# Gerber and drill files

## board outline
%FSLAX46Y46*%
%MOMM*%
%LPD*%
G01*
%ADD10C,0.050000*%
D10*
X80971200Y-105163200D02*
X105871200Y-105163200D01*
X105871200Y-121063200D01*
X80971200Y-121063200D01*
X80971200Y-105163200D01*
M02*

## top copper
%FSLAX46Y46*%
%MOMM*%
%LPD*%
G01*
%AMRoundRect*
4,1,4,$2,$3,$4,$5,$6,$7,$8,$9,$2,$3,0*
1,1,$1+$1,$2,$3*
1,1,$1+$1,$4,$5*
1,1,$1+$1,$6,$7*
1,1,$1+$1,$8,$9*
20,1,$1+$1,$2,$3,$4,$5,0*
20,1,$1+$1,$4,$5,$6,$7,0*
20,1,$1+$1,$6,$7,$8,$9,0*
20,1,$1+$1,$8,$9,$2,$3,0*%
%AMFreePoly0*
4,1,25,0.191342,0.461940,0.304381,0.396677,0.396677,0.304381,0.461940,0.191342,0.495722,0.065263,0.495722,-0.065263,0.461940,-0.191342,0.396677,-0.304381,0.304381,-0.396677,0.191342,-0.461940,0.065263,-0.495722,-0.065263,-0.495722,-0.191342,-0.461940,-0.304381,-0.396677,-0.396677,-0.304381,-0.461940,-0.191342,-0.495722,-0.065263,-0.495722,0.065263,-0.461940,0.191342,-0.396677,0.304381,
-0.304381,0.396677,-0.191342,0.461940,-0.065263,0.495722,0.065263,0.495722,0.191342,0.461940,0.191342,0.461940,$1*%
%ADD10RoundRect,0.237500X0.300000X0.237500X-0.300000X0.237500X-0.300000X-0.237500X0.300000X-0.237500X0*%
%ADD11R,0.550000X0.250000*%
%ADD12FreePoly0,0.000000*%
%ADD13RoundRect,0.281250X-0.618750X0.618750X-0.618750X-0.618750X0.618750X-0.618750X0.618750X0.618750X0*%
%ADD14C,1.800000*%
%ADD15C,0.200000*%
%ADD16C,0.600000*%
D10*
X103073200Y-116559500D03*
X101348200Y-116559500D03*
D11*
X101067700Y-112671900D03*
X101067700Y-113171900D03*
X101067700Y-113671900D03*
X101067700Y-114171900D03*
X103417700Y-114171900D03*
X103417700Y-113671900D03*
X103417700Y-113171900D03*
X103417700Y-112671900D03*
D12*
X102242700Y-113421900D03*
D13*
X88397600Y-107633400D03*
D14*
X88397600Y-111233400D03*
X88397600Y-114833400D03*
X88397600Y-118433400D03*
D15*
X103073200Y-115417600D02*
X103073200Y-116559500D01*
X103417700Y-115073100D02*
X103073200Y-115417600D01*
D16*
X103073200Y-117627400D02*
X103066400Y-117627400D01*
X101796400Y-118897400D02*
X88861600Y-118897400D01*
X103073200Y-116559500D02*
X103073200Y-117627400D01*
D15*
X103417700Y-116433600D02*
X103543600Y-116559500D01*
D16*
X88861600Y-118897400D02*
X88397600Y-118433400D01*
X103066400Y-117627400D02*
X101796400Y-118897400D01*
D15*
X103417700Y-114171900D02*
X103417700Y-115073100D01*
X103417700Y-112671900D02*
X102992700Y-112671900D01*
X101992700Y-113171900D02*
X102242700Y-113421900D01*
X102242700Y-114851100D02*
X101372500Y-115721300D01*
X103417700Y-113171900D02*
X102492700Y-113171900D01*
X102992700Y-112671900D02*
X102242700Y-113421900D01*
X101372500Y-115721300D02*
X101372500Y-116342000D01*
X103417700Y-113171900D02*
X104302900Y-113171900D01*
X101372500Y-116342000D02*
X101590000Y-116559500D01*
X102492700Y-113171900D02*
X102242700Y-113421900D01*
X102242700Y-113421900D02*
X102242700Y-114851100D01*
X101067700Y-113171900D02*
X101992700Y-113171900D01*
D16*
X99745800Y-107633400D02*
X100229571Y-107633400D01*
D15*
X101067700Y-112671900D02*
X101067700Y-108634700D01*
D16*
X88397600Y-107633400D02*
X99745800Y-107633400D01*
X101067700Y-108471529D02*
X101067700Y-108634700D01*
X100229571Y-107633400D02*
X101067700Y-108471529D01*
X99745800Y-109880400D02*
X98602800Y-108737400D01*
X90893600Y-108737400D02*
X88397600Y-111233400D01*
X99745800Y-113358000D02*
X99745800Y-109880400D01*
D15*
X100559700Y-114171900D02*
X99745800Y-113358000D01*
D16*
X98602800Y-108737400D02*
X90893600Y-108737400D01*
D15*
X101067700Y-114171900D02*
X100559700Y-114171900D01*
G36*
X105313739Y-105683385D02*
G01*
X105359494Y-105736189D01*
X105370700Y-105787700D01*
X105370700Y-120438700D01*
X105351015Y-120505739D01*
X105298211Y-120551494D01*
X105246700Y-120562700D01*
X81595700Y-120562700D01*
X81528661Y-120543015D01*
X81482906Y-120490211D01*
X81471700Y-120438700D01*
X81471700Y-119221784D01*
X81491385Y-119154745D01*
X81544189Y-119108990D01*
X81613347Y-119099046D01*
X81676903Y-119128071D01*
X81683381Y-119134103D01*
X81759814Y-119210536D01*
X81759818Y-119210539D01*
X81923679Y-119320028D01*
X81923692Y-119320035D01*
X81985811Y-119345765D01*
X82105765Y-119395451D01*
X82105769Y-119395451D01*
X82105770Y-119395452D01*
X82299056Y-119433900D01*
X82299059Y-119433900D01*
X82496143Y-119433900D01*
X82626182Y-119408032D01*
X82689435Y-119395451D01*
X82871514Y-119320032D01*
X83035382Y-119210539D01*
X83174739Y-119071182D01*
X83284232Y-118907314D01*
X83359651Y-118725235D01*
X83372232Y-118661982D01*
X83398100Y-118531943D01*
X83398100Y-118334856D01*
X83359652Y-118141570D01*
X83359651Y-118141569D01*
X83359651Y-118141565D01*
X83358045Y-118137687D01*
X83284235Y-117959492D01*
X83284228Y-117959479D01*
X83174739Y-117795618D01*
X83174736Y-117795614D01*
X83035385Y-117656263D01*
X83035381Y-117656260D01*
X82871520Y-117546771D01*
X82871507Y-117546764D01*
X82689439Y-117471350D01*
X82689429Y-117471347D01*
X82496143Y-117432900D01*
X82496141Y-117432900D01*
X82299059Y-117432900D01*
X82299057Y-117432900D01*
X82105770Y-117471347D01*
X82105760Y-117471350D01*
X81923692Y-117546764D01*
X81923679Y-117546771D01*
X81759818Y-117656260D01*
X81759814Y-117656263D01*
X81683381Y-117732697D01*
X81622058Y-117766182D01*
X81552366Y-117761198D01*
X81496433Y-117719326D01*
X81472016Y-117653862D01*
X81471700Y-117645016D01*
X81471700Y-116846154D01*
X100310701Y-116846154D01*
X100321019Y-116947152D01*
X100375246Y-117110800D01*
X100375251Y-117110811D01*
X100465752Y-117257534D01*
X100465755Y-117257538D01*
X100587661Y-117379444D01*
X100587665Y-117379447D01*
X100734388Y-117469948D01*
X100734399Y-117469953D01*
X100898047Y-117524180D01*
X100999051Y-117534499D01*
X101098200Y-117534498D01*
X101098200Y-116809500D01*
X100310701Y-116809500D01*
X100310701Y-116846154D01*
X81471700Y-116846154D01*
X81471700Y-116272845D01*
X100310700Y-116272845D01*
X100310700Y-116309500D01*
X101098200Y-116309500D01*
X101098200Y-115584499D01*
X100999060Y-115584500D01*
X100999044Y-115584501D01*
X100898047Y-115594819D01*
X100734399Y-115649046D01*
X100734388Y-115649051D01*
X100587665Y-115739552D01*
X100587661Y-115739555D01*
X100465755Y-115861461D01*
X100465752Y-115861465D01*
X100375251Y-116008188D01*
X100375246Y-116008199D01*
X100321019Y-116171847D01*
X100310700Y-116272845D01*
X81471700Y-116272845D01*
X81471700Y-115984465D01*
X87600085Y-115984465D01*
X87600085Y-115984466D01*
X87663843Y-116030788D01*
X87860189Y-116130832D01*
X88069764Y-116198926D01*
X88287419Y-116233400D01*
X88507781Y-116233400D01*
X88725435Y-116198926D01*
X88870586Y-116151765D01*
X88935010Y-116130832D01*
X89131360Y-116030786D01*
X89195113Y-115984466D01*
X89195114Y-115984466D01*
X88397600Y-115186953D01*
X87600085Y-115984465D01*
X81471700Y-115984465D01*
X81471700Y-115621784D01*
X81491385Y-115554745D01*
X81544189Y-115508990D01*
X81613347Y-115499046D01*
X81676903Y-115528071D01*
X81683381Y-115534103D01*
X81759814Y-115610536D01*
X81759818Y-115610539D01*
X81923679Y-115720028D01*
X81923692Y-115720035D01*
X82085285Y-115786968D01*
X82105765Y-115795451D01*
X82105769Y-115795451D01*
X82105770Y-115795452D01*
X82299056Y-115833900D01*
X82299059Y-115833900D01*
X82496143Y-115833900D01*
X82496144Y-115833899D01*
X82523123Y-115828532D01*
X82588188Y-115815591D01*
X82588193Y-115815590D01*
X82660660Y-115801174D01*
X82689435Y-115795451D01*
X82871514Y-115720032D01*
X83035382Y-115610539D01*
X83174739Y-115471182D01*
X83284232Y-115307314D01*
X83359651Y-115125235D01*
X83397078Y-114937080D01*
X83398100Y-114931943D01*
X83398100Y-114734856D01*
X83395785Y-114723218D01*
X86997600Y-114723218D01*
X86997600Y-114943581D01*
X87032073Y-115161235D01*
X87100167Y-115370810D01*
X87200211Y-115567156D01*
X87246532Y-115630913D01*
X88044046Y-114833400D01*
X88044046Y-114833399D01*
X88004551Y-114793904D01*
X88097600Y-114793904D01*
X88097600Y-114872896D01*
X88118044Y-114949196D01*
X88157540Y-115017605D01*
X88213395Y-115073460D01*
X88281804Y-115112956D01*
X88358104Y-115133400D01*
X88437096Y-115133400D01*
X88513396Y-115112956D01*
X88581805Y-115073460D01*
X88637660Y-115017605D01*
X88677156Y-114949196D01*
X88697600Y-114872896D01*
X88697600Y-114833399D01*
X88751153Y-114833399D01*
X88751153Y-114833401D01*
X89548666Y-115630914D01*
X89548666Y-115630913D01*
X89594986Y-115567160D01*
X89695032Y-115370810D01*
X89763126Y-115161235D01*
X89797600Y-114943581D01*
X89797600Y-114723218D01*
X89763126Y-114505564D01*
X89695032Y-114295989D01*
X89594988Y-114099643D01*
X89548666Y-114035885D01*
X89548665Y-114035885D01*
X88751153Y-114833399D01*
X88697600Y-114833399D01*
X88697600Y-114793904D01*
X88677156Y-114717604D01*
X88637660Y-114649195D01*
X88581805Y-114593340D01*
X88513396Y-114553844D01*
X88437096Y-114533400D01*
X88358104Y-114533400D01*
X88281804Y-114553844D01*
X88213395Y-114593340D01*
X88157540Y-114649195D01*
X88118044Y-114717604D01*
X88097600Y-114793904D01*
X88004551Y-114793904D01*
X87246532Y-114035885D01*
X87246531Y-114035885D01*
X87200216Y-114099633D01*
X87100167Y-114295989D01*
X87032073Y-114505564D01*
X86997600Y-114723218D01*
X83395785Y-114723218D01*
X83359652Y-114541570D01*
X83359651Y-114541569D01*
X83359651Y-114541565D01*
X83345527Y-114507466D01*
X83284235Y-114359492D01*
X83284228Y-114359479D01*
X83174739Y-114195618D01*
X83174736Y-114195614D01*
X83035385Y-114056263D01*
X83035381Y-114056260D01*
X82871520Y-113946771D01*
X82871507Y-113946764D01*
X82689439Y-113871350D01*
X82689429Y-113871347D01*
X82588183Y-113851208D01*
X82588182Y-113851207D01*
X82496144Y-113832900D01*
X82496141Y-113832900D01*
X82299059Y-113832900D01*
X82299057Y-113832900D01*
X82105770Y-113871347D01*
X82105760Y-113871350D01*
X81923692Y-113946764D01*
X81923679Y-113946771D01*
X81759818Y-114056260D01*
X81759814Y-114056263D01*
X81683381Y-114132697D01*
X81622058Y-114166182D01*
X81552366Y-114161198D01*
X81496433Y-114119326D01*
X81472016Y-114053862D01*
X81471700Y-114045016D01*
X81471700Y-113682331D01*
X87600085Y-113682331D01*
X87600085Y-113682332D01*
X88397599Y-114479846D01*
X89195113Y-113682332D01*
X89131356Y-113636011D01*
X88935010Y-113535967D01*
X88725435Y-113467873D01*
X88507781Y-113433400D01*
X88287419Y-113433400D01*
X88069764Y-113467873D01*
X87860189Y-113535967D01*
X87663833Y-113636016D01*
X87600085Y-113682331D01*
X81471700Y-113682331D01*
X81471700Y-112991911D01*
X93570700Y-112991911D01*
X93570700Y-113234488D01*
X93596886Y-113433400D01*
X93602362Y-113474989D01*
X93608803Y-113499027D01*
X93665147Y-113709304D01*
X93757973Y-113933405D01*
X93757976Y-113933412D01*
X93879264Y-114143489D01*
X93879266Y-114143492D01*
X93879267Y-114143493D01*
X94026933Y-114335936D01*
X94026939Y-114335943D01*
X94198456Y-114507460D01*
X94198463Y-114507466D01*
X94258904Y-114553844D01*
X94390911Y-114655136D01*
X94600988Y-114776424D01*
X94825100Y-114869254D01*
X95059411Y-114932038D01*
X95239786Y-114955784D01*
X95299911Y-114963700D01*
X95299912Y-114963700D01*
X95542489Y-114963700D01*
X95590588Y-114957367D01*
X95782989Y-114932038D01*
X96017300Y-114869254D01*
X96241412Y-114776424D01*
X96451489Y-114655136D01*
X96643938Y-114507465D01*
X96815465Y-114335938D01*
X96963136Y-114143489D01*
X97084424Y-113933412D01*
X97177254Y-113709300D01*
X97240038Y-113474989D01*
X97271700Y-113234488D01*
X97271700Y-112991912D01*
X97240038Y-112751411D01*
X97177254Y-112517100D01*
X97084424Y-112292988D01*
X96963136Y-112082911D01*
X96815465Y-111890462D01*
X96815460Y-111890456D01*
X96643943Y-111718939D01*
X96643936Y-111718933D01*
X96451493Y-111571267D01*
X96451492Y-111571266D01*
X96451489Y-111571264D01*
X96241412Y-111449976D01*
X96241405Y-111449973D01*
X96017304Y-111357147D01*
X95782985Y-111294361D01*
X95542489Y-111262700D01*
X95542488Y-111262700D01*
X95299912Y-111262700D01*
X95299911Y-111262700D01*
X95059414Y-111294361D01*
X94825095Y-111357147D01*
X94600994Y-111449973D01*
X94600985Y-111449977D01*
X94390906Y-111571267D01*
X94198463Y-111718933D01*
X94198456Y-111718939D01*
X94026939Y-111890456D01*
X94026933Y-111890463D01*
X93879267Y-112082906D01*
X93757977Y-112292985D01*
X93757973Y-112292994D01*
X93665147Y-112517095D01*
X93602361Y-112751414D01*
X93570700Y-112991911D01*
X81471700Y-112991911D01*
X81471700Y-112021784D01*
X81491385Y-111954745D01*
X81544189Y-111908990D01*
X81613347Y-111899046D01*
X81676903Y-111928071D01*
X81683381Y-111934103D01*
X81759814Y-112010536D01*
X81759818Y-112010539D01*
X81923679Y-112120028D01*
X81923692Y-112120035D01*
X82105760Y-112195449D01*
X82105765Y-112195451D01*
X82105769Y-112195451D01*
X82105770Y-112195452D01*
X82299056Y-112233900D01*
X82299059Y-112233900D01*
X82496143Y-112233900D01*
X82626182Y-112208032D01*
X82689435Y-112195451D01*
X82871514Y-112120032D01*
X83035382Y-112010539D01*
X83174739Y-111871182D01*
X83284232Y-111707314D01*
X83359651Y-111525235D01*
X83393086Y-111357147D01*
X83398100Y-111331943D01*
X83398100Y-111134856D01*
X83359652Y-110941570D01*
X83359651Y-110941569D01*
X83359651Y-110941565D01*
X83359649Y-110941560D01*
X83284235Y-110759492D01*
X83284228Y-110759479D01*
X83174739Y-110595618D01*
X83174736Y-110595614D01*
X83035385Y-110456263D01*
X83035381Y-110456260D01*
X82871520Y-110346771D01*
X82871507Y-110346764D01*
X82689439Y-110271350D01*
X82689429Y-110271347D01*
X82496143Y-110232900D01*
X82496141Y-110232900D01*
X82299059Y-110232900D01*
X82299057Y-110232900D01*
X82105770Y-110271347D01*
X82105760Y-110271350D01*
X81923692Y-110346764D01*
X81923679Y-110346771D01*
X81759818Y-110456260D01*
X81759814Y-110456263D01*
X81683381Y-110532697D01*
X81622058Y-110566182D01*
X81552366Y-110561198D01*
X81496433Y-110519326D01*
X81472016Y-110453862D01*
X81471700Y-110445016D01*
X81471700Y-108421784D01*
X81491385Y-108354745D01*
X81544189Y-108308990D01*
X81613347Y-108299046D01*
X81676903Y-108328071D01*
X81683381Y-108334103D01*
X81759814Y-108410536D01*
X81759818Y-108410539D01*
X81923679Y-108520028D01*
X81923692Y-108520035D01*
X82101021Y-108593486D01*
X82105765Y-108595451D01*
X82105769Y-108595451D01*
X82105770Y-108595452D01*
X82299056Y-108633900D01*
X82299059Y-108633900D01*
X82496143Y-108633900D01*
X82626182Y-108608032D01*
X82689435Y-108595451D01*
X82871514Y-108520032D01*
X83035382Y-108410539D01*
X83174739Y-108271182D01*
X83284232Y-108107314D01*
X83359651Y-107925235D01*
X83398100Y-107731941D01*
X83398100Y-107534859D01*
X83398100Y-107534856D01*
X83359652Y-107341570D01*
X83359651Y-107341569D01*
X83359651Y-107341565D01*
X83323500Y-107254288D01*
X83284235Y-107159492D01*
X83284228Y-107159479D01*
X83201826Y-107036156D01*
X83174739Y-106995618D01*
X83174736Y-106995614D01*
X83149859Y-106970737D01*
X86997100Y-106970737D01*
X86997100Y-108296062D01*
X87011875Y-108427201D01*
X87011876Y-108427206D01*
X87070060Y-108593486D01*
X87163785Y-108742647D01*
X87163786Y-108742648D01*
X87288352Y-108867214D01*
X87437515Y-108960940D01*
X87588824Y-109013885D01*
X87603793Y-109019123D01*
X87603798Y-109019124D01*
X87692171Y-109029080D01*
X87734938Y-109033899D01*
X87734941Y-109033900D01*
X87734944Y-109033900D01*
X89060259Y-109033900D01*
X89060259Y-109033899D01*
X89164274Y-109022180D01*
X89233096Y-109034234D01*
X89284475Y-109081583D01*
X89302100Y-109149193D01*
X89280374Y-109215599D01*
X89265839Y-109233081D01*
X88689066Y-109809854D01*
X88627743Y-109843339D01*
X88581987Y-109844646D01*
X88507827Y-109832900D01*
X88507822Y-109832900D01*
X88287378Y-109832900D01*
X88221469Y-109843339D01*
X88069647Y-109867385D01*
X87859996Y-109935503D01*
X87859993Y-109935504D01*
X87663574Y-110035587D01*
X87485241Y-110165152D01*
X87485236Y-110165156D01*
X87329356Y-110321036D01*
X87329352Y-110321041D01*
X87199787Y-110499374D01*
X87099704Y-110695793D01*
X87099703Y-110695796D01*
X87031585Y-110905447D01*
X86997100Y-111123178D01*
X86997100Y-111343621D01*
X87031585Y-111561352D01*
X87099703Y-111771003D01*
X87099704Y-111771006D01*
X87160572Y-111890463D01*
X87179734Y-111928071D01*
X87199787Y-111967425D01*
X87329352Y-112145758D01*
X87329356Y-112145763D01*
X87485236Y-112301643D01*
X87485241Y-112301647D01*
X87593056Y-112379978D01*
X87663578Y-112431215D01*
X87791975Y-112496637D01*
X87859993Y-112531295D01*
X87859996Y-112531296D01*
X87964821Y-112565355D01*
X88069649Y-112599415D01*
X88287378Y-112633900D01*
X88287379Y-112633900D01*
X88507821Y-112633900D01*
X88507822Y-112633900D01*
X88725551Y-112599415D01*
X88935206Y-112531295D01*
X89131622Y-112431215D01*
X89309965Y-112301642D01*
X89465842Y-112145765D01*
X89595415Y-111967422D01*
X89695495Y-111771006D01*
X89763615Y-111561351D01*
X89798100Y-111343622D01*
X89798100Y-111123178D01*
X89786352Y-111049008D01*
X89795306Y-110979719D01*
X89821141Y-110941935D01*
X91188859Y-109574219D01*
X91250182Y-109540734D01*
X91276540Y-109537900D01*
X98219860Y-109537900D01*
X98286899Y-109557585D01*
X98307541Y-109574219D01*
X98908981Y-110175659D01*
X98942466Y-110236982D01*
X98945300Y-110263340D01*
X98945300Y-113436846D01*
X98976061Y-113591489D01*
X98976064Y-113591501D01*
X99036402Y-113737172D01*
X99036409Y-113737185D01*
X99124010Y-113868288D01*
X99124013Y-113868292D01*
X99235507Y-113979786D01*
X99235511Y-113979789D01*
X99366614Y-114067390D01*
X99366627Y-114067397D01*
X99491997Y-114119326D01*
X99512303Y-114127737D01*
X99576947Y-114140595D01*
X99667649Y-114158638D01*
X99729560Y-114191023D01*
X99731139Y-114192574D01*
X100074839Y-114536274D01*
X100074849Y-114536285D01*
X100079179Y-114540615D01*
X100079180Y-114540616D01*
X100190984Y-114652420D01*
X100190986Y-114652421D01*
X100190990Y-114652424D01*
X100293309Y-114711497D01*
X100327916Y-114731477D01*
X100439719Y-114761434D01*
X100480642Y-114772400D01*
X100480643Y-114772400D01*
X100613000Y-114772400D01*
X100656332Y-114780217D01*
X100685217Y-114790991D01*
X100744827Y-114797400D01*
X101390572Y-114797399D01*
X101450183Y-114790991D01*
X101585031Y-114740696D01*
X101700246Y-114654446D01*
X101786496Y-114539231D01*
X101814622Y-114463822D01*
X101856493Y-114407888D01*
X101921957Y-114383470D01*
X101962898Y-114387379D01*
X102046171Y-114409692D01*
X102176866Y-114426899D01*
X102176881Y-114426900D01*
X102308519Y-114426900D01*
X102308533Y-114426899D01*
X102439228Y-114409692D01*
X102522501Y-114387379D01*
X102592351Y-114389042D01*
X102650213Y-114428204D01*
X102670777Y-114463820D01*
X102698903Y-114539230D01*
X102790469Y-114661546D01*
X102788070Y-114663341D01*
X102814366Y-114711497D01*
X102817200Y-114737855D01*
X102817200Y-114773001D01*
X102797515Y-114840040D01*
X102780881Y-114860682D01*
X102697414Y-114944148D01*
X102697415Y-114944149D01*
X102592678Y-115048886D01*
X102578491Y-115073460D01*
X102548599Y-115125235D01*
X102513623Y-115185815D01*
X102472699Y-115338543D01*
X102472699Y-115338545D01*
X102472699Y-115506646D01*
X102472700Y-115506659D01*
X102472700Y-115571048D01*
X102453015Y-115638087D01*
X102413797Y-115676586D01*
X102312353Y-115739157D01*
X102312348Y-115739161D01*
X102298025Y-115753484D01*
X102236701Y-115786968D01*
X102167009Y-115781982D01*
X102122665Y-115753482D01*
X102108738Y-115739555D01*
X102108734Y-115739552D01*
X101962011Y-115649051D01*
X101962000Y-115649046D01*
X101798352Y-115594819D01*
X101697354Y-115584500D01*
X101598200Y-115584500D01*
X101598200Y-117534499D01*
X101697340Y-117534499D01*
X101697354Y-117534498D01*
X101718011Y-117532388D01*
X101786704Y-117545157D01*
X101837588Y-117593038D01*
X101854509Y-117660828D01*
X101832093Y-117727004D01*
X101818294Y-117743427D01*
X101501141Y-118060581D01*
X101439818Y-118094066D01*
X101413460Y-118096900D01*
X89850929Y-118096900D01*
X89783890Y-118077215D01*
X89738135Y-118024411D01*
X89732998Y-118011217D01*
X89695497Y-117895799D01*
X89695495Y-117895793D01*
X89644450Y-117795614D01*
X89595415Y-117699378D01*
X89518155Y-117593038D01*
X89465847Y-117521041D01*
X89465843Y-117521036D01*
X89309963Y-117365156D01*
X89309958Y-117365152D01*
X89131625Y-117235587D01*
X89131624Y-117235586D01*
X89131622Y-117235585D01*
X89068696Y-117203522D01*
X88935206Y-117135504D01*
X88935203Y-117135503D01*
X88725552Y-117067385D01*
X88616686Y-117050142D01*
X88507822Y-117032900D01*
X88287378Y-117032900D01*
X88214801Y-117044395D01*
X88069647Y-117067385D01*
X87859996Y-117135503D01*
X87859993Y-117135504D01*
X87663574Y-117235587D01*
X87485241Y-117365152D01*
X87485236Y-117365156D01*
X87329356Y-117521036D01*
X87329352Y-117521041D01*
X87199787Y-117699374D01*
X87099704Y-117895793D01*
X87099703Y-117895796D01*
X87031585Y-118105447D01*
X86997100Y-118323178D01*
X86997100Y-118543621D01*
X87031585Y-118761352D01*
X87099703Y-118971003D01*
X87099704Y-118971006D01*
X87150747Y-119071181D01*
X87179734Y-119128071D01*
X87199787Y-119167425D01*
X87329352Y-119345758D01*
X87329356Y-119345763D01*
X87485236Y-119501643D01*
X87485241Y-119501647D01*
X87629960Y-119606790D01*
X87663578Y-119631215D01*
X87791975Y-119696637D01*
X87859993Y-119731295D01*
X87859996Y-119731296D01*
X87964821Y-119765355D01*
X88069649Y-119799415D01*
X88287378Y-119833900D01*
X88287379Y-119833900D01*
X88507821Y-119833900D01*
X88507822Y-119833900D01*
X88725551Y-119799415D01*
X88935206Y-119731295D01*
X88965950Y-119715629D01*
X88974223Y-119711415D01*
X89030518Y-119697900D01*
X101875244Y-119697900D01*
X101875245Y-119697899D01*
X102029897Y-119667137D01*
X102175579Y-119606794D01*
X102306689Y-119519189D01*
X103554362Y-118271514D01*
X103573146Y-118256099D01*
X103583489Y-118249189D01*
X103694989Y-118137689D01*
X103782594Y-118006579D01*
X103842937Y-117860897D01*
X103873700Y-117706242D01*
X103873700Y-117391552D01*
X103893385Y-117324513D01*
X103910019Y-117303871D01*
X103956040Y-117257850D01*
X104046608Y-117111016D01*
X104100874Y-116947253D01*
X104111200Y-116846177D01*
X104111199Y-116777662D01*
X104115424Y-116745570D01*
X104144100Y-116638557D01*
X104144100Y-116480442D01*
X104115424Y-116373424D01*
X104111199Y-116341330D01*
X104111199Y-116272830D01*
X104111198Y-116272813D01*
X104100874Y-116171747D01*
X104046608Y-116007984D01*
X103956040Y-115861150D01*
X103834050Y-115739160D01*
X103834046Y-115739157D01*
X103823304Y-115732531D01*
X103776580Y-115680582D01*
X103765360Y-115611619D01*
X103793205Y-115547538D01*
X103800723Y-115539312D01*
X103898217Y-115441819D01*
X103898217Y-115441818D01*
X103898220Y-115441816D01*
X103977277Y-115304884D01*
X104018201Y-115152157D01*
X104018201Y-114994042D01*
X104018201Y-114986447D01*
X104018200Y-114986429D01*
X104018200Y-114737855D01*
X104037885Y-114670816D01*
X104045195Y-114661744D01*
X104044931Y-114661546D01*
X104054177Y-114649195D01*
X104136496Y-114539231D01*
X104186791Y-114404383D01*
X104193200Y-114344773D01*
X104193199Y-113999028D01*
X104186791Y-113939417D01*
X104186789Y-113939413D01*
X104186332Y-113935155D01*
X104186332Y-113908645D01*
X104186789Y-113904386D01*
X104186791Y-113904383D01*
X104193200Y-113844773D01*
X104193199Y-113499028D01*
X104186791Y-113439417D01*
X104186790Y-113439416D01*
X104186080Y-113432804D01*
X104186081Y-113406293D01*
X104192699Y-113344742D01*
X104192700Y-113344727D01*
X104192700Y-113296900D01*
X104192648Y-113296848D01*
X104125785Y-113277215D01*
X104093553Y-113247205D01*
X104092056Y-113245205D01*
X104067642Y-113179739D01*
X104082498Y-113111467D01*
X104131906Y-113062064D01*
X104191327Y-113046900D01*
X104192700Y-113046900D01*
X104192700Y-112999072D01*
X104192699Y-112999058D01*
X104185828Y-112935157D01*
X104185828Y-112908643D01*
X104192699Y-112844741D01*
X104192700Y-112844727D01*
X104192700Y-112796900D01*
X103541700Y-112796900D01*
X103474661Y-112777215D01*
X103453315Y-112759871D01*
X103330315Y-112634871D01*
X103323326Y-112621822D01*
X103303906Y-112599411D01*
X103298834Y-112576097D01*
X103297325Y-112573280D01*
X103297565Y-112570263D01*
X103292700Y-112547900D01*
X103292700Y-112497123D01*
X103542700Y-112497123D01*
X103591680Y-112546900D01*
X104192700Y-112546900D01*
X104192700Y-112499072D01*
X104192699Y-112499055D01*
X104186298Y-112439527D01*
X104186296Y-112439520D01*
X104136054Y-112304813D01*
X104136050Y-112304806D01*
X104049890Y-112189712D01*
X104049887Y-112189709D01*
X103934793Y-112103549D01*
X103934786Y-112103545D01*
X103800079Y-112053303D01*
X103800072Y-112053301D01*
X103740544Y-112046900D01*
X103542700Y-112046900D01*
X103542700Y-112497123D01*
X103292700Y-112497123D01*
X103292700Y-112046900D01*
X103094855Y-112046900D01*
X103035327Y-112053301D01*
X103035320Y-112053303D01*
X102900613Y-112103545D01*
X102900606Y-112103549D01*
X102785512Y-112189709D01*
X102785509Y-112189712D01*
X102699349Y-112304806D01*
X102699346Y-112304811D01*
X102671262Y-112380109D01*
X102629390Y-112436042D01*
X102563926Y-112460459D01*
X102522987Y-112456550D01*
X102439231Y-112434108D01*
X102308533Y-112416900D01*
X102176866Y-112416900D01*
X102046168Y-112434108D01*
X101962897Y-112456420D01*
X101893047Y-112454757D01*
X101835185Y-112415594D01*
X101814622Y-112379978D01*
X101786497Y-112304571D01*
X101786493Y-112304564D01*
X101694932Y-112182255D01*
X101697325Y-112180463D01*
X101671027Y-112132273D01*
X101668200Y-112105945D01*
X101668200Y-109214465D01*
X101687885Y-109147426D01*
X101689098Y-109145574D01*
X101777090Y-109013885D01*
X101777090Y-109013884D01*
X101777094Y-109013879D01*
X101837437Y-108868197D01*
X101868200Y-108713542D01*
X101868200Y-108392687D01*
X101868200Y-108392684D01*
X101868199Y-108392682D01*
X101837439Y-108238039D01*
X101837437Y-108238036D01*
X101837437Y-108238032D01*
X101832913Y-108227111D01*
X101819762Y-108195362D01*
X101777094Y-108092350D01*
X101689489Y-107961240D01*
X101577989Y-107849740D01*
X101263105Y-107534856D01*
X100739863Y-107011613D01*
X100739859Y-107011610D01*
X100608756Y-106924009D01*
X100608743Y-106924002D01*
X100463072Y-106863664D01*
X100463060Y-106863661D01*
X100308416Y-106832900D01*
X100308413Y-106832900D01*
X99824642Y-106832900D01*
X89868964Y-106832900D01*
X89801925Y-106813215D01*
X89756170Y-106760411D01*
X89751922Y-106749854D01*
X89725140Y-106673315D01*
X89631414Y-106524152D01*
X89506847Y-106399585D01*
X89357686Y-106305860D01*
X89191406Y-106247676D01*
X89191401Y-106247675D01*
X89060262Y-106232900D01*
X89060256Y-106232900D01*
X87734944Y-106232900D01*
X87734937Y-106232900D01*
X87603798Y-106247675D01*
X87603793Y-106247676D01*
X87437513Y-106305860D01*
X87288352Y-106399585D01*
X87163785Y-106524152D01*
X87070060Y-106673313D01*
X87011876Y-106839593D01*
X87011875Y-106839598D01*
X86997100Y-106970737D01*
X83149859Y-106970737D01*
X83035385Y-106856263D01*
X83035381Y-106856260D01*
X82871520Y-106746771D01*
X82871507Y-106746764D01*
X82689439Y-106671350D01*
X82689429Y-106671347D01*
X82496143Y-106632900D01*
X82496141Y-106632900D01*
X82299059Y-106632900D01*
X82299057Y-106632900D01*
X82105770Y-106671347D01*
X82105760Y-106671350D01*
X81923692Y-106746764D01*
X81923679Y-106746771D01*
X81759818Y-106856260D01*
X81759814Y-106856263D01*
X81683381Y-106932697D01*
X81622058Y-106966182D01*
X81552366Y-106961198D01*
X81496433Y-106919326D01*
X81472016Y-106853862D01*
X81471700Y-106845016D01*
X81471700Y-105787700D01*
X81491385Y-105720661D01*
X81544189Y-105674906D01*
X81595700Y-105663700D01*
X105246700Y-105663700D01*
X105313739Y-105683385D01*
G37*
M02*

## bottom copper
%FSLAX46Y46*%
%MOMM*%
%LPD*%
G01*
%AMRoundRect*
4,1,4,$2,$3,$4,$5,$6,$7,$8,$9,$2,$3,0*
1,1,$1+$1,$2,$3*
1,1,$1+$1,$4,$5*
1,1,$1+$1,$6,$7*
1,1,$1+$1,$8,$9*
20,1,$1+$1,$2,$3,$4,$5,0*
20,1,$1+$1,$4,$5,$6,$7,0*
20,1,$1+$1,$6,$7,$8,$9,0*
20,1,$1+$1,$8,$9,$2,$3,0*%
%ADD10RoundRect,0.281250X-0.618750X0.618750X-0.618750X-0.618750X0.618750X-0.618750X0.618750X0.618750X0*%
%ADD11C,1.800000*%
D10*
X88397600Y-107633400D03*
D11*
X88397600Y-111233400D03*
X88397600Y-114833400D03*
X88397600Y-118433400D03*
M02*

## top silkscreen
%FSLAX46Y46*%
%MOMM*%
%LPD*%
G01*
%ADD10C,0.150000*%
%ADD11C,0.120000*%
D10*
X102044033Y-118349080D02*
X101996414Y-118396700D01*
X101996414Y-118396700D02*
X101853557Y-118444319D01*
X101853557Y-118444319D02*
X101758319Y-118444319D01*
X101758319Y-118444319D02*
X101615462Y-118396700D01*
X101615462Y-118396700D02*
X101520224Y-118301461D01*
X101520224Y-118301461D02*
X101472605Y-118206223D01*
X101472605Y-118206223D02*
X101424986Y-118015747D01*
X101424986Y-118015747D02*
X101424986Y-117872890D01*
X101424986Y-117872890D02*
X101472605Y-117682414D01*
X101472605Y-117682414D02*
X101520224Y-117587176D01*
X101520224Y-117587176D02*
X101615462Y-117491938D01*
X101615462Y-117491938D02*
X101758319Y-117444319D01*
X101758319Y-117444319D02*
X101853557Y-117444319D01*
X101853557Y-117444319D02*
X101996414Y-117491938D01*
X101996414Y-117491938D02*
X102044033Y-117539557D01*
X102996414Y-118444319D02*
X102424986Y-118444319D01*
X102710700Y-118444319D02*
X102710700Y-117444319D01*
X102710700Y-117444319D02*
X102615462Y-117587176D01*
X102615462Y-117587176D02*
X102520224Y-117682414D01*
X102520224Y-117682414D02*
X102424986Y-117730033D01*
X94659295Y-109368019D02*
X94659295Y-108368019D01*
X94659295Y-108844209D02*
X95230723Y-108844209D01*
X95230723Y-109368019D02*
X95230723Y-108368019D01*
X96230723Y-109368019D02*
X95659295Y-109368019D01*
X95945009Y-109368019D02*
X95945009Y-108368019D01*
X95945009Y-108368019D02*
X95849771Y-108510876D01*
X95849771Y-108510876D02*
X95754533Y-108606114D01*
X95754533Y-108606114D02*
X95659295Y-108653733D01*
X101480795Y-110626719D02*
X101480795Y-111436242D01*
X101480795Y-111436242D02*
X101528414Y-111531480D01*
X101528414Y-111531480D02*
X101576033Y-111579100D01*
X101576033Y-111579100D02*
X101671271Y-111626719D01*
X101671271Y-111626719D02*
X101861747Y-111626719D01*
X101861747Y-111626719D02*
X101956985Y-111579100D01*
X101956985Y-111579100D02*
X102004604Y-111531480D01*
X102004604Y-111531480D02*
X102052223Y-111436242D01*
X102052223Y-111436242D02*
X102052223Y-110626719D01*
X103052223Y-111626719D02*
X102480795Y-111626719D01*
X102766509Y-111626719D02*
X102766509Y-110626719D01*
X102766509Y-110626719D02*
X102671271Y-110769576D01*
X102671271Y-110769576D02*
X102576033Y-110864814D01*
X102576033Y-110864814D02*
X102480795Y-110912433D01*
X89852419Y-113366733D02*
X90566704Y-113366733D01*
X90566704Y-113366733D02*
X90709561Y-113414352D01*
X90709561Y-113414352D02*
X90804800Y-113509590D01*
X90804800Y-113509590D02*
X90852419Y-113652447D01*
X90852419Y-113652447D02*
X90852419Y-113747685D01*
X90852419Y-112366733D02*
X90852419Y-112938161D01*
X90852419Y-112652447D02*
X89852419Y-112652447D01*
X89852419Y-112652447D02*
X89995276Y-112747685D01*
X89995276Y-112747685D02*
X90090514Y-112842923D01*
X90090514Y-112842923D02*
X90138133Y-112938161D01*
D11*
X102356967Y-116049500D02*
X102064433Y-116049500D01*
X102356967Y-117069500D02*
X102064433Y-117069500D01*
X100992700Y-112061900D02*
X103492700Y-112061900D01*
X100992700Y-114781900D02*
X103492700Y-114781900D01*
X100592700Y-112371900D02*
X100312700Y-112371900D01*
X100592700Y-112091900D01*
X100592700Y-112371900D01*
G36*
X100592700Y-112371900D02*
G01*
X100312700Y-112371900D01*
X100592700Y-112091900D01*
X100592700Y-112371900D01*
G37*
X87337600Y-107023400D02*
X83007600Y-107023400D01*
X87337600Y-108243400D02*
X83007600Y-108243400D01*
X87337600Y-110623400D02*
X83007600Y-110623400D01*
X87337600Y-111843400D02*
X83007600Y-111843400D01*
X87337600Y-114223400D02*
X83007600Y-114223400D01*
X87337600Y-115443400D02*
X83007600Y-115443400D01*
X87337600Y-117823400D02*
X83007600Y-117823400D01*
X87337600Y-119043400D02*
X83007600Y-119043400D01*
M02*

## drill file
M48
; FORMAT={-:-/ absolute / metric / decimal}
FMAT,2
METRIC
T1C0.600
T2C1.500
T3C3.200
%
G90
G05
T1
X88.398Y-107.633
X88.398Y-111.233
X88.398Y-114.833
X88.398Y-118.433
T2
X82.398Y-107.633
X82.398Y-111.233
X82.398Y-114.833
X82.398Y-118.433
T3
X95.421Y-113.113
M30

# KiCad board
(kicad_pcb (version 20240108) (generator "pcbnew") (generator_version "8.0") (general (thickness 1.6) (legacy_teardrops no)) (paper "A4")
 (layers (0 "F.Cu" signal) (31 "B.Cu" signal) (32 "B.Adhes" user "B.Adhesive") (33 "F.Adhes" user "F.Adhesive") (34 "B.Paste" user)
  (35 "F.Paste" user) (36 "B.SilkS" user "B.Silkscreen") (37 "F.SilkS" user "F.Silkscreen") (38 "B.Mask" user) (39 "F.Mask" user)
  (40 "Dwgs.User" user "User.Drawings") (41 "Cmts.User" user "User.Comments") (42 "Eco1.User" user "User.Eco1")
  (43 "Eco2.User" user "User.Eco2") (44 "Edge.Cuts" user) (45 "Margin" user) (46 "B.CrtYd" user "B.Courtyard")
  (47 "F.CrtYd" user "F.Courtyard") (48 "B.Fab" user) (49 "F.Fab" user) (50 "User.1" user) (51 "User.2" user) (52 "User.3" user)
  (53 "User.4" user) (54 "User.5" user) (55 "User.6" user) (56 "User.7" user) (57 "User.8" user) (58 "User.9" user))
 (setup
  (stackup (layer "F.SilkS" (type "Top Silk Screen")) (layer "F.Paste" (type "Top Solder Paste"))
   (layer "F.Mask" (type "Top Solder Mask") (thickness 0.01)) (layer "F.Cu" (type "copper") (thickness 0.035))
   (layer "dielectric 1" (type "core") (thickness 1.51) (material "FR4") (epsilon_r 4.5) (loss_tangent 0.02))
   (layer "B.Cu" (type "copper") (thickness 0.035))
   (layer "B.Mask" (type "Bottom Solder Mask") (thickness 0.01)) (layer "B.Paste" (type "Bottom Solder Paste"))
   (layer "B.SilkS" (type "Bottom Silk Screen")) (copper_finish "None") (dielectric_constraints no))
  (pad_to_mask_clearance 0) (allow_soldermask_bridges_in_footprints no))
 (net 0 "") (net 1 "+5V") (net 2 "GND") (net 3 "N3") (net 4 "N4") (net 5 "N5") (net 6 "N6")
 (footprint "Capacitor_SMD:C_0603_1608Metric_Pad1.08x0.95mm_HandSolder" (layer "F.Cu") (at 102.2107 116.5595 180)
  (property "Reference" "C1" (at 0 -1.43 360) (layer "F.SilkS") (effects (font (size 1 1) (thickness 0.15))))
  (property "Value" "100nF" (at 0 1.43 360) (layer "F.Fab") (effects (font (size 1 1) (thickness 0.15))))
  (fp_line (start -0.146267 0.51) (end 0.146267 0.51) (stroke (width 0.12) (type solid)) (layer "F.SilkS"))
  (fp_line (start -0.146267 -0.51) (end 0.146267 -0.51) (stroke (width 0.12) (type solid)) (layer "F.SilkS"))
  (pad "1" smd roundrect (at -0.8625 0 180) (size 1.075 0.95) (layers "F.Cu" "F.Paste" "F.Mask") (roundrect_rratio 0.25) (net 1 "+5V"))
  (pad "2" smd roundrect (at 0.8625 0 180) (size 1.075 0.95) (layers "F.Cu" "F.Paste" "F.Mask") (roundrect_rratio 0.25) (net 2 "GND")))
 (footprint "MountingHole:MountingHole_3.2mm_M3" (layer "F.Cu") (at 95.4212 113.1132)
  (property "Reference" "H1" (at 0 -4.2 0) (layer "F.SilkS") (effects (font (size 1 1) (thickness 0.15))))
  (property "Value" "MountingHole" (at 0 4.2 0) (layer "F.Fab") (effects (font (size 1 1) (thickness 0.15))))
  (pad "" np_thru_hole circle (at 0 0) (size 3.2 3.2) (drill 3.2) (layers "*.Cu" "*.Mask")))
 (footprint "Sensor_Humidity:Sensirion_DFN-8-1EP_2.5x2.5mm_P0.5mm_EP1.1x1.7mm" (layer "F.Cu") (at 102.2427 113.4219)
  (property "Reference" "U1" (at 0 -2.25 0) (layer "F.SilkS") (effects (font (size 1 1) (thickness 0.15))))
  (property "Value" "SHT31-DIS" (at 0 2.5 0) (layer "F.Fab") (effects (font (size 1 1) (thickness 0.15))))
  (fp_line (start -1.25 -1.36) (end 1.25 -1.36) (stroke (width 0.12) (type solid)) (layer "F.SilkS"))
  (fp_line (start -1.25 1.36) (end 1.25 1.36) (stroke (width 0.12) (type solid)) (layer "F.SilkS"))
  (fp_poly
   (pts (xy -1.65 -1.05) (xy -1.93 -1.05) (xy -1.65 -1.33) (xy -1.65 -1.05)) (stroke (width 0.12) (type solid)) (fill solid)
   (layer "F.SilkS"))
  (pad "" smd custom (at 0 0) (size 0.9 0.9) (layers "F.Paste") (zone_connect 0) (thermal_bridge_angle 45)
   (options (clearance outline) (anchor rect)) (primitives))
  (pad "1" smd rect (at -1.175 -0.75) (size 0.55 0.25) (layers "F.Cu" "F.Paste" "F.Mask") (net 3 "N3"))
  (pad "2" smd rect (at -1.175 -0.25) (size 0.55 0.25) (layers "F.Cu" "F.Paste" "F.Mask") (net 2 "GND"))
  (pad "3" smd rect (at -1.175 0.25) (size 0.55 0.25) (layers "F.Cu" "F.Paste" "F.Mask") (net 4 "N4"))
  (pad "4" smd rect (at -1.175 0.75 180) (size 0.55 0.25) (layers "F.Cu" "F.Paste" "F.Mask") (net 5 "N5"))
  (pad "5" smd rect (at 1.175 0.75) (size 0.55 0.25) (layers "F.Cu" "F.Paste" "F.Mask") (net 1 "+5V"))
  (pad "6" smd rect (at 1.175 0.25) (size 0.55 0.25) (layers "F.Cu" "F.Paste" "F.Mask") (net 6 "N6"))
  (pad "7" smd rect (at 1.175 -0.25) (size 0.55 0.25) (layers "F.Cu" "F.Paste" "F.Mask") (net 2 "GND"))
  (pad "8" smd rect (at 1.175 -0.75) (size 0.55 0.25) (layers "F.Cu" "F.Paste" "F.Mask") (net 2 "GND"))
  (pad "9" smd custom (at 0 0) (size 1 1) (layers "F.Cu" "F.Mask") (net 2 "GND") (zone_connect 0)
   (options (clearance outline) (anchor circle)) (primitives)))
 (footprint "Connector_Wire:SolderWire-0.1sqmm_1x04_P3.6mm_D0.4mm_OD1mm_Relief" (layer "F.Cu") (at 88.3976 107.6334 -90)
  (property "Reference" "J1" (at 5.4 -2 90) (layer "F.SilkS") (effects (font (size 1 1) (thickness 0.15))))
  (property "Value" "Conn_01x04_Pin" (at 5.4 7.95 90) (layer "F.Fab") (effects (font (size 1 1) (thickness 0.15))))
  (fp_line (start -0.61 1.06) (end -0.61 5.39) (stroke (width 0.12) (type solid)) (layer "F.SilkS"))
  (fp_line (start 0.61 1.06) (end 0.61 5.39) (stroke (width 0.12) (type solid)) (layer "F.SilkS"))
  (fp_line (start 2.99 1.06) (end 2.99 5.39) (stroke (width 0.12) (type solid)) (layer "F.SilkS"))
  (fp_line (start 4.21 1.06) (end 4.21 5.39) (stroke (width 0.12) (type solid)) (layer "F.SilkS"))
  (fp_line (start 6.59 1.06) (end 6.59 5.39) (stroke (width 0.12) (type solid)) (layer "F.SilkS"))
  (fp_line (start 7.81 1.06) (end 7.81 5.39) (stroke (width 0.12) (type solid)) (layer "F.SilkS"))
  (fp_line (start 10.19 1.06) (end 10.19 5.39) (stroke (width 0.12) (type solid)) (layer "F.SilkS"))
  (fp_line (start 11.41 1.06) (end 11.41 5.39) (stroke (width 0.12) (type solid)) (layer "F.SilkS"))
  (pad "" np_thru_hole circle (at 0 6 270) (size 1.5 1.5) (drill 1.5) (layers "F&B.Cu" "*.Mask"))
  (pad "" np_thru_hole circle (at 3.6 6 270) (size 1.5 1.5) (drill 1.5) (layers "*.Cu" "*.Mask"))
  (pad "" np_thru_hole circle (at 7.2 6 270) (size 1.5 1.5) (drill 1.5) (layers "*.Cu" "*.Mask"))
  (pad "" np_thru_hole circle (at 10.8 6 270) (size 1.5 1.5) (drill 1.5) (layers "*.Cu" "*.Mask"))
  (pad "1" thru_hole roundrect (at 0 0 270) (size 1.8 1.8) (drill 0.6) (layers "*.Cu" "*.Mask") (remove_unused_layers no)
   (roundrect_rratio 0.15625) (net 3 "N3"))
  (pad "2" thru_hole circle (at 3.6 0 270) (size 1.8 1.8) (drill 0.6) (layers "*.Cu" "*.Mask") (remove_unused_layers no) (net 5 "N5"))
  (pad "3" thru_hole circle (at 7.2 0 270) (size 1.8 1.8) (drill 0.6) (layers "*.Cu" "*.Mask") (remove_unused_layers no) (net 2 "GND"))
  (pad "4" thru_hole circle (at 10.8 0 270) (size 1.8 1.8) (drill 0.6) (layers "*.Cu" "*.Mask") (remove_unused_layers no) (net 1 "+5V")))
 (gr_rect (start 80.9712 105.1632) (end 105.8712 121.0632) (stroke (width 0.05) (type default)) (fill none) (layer "Edge.Cuts"))
 (segment (start 103.0732 115.4176) (end 103.0732 116.5595) (width 0.2) (layer "F.Cu") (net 1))
 (segment (start 103.4177 115.0731) (end 103.0732 115.4176) (width 0.2) (layer "F.Cu") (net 1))
 (segment (start 103.0732 117.6274) (end 103.0664 117.6274) (width 0.6) (layer "F.Cu") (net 1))
 (segment (start 101.7964 118.8974) (end 88.8616 118.8974) (width 0.6) (layer "F.Cu") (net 1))
 (segment (start 103.0732 116.5595) (end 103.0732 117.6274) (width 0.6) (layer "F.Cu") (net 1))
 (segment (start 103.4177 116.4336) (end 103.5436 116.5595) (width 0.2) (layer "F.Cu") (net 1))
 (segment (start 88.8616 118.8974) (end 88.3976 118.4334) (width 0.6) (layer "F.Cu") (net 1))
 (segment (start 103.0664 117.6274) (end 101.7964 118.8974) (width 0.6) (layer "F.Cu") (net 1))
 (segment (start 103.4177 114.1719) (end 103.4177 115.0731) (width 0.2) (layer "F.Cu") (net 1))
 (segment (start 103.4177 112.6719) (end 102.9927 112.6719) (width 0.2) (layer "F.Cu") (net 2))
 (segment (start 101.9927 113.1719) (end 102.2427 113.4219) (width 0.2) (layer "F.Cu") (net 2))
 (segment (start 102.2427 114.8511) (end 101.3725 115.7213) (width 0.2) (layer "F.Cu") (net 2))
 (segment (start 103.4177 113.1719) (end 102.4927 113.1719) (width 0.2) (layer "F.Cu") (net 2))
 (segment (start 102.9927 112.6719) (end 102.2427 113.4219) (width 0.2) (layer "F.Cu") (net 2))
 (segment (start 101.3725 115.7213) (end 101.3725 116.342) (width 0.2) (layer "F.Cu") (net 2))
 (segment (start 103.4177 113.1719) (end 104.3029 113.1719) (width 0.2) (layer "F.Cu") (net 2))
 (segment (start 101.3725 116.342) (end 101.59 116.5595) (width 0.2) (layer "F.Cu") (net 2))
 (segment (start 102.4927 113.1719) (end 102.2427 113.4219) (width 0.2) (layer "F.Cu") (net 2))
 (segment (start 102.2427 113.4219) (end 102.2427 114.8511) (width 0.2) (layer "F.Cu") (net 2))
 (segment (start 101.0677 113.1719) (end 101.9927 113.1719) (width 0.2) (layer "F.Cu") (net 2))
 (segment (start 99.7458 107.6334) (end 100.229571 107.6334) (width 0.6) (layer "F.Cu") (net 3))
 (segment (start 101.0677 112.6719) (end 101.0677 108.6347) (width 0.2) (layer "F.Cu") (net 3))
 (segment (start 88.3976 107.6334) (end 99.7458 107.6334) (width 0.6) (layer "F.Cu") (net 3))
 (segment (start 101.0677 108.471529) (end 101.0677 108.6347) (width 0.6) (layer "F.Cu") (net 3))
 (segment (start 100.229571 107.6334) (end 101.0677 108.471529) (width 0.6) (layer "F.Cu") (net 3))
 (segment (start 99.7458 109.8804) (end 98.6028 108.7374) (width 0.6) (layer "F.Cu") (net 5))
 (segment (start 90.8936 108.7374) (end 88.3976 111.2334) (width 0.6) (layer "F.Cu") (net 5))
 (segment (start 99.7458 113.358) (end 99.7458 109.8804) (width 0.6) (layer "F.Cu") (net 5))
 (segment (start 100.5597 114.1719) (end 99.7458 113.358) (width 0.2) (layer "F.Cu") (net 5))
 (segment (start 98.6028 108.7374) (end 90.8936 108.7374) (width 0.6) (layer "F.Cu") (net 5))
 (segment (start 101.0677 114.1719) (end 100.5597 114.1719) (width 0.2) (layer "F.Cu") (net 5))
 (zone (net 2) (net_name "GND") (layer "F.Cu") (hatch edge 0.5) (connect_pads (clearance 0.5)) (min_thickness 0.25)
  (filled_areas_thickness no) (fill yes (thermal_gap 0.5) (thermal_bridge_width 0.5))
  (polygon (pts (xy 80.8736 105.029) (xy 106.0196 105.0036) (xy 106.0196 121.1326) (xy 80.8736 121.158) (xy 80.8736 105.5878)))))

